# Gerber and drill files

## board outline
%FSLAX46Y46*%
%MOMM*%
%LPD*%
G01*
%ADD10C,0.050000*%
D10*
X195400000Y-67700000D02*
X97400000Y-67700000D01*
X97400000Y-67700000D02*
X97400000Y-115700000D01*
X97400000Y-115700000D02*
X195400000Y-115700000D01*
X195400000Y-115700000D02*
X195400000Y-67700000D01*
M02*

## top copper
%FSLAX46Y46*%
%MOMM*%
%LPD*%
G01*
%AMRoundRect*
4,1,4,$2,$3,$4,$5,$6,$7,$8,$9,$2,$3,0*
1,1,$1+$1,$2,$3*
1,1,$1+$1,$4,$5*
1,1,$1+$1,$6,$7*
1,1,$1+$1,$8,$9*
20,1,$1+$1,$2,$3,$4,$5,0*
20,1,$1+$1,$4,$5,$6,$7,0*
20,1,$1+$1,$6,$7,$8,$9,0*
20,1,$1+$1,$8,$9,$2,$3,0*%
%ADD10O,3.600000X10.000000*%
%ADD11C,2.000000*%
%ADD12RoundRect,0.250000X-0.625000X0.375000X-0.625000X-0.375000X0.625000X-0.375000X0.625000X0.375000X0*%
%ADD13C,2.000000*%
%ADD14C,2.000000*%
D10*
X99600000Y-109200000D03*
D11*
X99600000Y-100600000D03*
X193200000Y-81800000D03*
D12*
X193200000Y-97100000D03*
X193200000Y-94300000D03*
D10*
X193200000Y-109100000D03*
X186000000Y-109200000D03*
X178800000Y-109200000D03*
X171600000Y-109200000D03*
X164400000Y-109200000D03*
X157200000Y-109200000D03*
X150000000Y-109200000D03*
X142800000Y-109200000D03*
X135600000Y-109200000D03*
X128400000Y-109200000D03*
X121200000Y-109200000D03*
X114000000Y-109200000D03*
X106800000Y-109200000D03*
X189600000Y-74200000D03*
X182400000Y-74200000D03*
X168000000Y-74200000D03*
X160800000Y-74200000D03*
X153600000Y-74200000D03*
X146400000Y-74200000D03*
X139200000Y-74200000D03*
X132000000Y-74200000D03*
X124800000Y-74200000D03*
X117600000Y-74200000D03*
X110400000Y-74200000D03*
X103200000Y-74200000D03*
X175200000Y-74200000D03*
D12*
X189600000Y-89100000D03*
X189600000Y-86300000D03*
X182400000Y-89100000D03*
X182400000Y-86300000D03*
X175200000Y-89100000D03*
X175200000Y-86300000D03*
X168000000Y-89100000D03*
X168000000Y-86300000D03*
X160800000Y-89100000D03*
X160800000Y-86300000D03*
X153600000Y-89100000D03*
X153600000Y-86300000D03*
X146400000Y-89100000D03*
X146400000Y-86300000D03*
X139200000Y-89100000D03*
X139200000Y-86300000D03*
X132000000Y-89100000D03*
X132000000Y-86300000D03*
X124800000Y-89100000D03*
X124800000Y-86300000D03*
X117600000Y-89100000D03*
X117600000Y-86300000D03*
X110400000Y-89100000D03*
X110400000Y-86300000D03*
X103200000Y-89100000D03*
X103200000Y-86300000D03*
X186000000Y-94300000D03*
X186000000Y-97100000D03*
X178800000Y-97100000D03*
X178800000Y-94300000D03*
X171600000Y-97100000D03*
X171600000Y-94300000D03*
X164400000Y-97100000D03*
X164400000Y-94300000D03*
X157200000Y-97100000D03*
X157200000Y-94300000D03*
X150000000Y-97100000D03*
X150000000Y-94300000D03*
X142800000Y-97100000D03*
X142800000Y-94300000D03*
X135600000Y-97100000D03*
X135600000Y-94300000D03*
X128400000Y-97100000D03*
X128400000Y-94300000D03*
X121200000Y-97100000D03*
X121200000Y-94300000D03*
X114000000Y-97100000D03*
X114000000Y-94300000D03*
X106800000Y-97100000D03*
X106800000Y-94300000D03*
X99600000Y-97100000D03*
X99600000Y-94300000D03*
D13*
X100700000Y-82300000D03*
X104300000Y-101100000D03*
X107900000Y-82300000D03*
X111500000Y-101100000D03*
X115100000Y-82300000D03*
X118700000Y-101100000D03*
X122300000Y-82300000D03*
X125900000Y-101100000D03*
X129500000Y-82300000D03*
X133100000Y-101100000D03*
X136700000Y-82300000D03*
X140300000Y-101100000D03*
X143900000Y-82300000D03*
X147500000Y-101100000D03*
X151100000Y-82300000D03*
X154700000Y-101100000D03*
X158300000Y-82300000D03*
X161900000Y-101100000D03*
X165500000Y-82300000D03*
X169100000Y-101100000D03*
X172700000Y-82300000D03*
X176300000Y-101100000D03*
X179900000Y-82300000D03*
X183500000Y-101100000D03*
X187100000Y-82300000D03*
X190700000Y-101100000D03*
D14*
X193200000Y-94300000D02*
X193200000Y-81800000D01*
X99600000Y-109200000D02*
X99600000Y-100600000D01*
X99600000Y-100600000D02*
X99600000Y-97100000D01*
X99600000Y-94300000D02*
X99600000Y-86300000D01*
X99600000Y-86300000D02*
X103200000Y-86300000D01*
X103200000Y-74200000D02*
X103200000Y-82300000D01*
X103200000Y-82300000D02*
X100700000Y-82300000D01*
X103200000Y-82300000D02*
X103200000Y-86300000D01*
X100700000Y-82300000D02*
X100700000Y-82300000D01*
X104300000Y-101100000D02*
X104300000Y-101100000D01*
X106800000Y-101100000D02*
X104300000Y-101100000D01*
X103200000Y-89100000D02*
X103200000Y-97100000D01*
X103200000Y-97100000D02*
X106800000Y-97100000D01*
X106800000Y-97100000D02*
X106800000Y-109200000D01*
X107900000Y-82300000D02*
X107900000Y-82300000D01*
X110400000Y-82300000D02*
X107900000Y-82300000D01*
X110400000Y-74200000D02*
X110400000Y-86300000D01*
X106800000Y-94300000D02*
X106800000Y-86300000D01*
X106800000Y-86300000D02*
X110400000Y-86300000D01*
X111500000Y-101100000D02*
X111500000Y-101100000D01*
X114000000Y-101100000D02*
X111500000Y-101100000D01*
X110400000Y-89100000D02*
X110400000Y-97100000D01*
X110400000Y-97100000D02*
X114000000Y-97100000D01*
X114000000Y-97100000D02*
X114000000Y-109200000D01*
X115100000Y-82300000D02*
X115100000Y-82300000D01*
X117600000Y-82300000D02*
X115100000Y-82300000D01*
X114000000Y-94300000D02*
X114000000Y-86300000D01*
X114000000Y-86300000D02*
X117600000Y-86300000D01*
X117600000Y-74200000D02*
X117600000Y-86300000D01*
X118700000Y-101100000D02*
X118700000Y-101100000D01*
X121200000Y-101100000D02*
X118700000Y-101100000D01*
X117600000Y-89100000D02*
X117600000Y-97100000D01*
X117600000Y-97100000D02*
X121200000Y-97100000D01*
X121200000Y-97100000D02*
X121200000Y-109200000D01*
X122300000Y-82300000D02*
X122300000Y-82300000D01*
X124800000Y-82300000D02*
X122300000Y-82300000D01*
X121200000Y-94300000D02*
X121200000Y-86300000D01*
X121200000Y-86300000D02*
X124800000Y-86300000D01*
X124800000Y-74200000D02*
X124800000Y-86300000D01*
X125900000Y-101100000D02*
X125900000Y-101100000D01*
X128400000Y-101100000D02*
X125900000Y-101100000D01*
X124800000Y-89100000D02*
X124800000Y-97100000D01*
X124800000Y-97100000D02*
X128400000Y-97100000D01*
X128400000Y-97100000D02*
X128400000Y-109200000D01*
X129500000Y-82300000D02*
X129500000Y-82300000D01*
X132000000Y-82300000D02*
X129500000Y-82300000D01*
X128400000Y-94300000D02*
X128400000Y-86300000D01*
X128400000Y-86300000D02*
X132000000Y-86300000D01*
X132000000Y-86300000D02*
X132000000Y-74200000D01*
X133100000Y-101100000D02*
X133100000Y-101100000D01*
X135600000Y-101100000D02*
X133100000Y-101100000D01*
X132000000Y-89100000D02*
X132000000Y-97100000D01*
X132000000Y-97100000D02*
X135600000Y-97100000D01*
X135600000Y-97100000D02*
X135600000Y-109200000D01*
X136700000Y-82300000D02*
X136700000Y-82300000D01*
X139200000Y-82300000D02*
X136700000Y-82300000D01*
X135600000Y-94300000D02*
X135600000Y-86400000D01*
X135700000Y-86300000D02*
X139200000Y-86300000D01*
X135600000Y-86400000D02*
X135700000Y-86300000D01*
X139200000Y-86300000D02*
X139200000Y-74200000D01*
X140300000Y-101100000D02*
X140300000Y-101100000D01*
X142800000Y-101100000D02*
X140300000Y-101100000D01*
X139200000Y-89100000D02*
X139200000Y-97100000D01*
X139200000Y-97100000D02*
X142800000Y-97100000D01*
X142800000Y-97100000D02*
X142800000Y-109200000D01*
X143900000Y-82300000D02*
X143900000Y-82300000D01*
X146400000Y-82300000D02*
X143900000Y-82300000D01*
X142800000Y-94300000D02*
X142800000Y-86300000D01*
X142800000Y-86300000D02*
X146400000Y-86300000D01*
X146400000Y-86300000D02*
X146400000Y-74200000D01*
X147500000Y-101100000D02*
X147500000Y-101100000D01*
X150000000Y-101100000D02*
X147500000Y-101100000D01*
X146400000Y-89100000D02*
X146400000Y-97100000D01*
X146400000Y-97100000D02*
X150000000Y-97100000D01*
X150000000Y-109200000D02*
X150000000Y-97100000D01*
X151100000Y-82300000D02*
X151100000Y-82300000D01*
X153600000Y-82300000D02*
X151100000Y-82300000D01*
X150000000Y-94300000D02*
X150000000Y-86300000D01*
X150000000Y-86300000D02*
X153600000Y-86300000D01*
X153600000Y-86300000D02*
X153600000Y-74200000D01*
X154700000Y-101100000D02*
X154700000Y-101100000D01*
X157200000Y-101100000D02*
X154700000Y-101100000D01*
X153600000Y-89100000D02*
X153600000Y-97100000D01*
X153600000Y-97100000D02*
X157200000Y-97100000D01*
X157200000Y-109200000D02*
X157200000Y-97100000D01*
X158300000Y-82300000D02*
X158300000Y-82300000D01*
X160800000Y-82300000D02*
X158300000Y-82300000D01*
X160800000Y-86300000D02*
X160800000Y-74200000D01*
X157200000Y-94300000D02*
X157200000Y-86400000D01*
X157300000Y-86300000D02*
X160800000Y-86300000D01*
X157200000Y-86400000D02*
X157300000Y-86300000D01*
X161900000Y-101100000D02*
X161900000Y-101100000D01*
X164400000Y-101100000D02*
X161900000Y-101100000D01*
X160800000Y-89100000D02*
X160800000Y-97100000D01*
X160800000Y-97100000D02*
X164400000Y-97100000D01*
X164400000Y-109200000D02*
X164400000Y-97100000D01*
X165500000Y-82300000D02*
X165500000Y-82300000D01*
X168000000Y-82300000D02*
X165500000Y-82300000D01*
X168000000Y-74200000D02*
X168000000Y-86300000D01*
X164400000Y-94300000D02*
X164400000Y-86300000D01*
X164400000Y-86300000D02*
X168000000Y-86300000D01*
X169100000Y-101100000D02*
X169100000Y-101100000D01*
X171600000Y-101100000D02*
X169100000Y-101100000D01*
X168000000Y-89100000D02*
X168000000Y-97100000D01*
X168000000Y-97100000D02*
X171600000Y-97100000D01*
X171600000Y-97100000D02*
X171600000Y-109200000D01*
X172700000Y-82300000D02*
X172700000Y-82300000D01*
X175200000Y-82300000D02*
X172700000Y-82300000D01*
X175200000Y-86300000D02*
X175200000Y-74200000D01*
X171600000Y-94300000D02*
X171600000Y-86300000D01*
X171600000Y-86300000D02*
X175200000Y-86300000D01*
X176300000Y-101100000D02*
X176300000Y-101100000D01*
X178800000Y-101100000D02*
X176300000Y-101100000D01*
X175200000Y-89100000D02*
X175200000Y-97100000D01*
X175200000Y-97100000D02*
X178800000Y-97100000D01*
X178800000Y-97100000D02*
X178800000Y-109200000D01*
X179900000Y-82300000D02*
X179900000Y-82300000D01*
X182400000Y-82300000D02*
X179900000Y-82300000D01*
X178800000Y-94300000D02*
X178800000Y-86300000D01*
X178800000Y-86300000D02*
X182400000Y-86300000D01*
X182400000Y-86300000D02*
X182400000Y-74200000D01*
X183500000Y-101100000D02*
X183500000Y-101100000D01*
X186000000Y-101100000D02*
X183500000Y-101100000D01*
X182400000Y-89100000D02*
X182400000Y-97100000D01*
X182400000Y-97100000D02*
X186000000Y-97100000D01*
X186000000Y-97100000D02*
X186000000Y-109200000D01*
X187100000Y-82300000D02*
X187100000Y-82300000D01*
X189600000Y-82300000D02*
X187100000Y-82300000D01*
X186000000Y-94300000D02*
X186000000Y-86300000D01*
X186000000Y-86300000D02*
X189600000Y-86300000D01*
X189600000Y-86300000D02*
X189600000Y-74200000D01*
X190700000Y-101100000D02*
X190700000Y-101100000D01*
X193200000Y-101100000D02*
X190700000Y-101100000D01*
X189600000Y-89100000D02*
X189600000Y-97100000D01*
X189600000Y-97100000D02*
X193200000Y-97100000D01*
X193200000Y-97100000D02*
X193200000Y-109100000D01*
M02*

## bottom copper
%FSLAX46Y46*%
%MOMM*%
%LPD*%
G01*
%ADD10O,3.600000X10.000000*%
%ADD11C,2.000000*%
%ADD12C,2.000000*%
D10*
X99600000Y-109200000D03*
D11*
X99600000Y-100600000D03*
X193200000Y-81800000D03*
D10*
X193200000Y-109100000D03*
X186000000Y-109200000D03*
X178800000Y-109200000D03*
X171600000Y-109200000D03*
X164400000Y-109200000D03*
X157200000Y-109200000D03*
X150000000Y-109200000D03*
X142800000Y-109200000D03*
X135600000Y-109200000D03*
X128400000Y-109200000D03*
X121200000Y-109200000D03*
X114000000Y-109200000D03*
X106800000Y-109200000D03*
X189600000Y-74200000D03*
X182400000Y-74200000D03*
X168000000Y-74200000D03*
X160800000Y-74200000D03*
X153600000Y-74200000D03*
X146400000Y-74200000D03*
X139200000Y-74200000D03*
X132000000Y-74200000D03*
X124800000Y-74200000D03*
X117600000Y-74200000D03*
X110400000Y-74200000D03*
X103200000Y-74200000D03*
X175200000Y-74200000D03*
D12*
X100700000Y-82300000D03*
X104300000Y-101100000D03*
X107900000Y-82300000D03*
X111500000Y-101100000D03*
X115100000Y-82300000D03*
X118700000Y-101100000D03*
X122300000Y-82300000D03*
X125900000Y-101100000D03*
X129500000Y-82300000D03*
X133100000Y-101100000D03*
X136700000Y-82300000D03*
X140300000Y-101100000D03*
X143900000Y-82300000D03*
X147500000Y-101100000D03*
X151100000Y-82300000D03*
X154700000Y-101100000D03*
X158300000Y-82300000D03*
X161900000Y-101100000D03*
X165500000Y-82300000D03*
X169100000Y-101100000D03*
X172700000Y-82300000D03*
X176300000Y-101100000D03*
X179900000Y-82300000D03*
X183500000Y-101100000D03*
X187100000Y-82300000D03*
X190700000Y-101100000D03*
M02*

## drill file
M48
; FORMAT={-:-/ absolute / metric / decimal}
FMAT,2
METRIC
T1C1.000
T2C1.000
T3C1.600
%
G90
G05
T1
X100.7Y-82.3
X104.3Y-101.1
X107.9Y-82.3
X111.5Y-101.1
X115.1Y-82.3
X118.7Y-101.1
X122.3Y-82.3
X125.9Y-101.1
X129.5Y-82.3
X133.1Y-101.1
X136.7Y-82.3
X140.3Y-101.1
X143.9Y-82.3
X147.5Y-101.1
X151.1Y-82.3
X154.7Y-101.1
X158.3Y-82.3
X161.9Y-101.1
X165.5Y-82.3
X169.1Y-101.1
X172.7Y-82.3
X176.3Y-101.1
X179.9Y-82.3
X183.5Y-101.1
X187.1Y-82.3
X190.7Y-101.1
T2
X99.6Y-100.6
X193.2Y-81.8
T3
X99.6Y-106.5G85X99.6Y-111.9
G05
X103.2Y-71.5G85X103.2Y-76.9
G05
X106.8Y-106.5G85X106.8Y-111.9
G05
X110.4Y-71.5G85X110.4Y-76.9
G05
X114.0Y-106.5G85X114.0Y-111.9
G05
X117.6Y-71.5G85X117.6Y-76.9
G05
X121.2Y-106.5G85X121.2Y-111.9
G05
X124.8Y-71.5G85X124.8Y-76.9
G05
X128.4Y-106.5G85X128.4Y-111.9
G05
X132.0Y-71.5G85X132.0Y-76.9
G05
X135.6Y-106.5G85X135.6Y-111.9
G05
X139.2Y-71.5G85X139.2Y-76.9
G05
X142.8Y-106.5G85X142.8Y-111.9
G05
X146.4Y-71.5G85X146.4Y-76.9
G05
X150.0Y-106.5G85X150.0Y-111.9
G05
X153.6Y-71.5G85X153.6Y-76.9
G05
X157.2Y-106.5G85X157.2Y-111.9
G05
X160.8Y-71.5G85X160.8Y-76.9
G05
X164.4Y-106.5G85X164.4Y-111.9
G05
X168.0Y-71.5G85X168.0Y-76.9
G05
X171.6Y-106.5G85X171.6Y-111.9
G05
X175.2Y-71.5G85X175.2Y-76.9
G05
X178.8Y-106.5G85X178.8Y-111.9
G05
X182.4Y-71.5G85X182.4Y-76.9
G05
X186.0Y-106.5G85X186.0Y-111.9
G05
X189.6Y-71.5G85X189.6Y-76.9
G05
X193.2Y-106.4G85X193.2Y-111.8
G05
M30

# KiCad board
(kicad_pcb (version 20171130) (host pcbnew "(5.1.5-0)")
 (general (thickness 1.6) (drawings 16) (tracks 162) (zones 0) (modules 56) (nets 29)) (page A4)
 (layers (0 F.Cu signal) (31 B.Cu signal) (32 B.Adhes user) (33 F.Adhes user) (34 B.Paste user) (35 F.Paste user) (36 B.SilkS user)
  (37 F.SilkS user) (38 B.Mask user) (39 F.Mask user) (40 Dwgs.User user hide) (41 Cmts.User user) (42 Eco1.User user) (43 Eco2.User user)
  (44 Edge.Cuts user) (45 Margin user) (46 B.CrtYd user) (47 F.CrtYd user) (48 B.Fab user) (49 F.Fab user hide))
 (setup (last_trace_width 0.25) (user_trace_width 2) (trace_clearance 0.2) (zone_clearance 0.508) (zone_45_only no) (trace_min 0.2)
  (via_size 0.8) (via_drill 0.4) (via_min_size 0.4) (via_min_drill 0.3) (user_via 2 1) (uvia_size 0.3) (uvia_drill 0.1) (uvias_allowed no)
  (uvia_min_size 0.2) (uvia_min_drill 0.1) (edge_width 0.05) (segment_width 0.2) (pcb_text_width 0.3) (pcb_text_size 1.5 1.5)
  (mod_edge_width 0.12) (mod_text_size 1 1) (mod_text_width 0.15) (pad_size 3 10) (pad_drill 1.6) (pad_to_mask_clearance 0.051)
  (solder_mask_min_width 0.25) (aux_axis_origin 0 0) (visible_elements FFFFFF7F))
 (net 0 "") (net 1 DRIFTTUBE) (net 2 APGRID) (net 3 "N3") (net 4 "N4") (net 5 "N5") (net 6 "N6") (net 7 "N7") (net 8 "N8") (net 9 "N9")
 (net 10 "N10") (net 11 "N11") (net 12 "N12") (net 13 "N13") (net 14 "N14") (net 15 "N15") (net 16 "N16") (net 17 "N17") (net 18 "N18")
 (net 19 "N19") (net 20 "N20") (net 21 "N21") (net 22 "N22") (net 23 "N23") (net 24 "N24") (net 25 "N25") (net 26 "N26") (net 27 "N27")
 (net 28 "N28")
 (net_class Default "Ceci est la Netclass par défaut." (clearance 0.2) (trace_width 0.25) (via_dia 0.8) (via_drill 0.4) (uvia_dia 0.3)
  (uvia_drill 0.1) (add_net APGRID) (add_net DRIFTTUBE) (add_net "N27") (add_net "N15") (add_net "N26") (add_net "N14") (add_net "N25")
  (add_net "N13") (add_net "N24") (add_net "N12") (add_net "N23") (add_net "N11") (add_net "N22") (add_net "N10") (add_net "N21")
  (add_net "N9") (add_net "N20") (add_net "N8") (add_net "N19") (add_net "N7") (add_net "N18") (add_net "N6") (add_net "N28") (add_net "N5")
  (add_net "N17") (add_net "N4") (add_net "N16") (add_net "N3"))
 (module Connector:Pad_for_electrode (layer F.Cu) (at 99.6 109.3)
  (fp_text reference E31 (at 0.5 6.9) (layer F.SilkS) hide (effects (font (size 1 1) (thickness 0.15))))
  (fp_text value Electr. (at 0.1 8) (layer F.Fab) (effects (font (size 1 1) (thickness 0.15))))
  (pad 1 thru_hole oval (at 0 -0.1) (size 3.6 10) (drill oval 1.6 7) (layers *.Cu *.Mask) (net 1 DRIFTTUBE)))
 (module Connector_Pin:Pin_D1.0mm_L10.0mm (layer F.Cu) (at 99.6 100.6)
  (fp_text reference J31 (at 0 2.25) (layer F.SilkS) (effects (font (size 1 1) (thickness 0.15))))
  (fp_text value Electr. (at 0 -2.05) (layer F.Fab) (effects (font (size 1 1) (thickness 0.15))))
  (pad 1 thru_hole circle (at 0 0) (size 2 2) (drill 1) (layers *.Cu *.Mask) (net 1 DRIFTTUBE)))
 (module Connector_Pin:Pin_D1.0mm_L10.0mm (layer F.Cu) (at 193.2 81.8)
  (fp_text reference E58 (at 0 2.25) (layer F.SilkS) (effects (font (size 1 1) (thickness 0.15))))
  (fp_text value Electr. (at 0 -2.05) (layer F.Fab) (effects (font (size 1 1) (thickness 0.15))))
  (pad 1 thru_hole circle (at 0 0) (size 2 2) (drill 1) (layers *.Cu *.Mask) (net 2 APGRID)))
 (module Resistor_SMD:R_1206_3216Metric (layer F.Cu) (at 193.2 95.7 270)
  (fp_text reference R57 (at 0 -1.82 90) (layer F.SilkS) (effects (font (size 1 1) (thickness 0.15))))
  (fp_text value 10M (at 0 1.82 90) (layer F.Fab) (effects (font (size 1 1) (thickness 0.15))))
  (pad 2 smd roundrect (at 1.4 0 270) (size 1.25 1.75) (layers F.Cu F.Paste F.Mask) (roundrect_rratio 0.2) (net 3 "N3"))
  (pad 1 smd roundrect (at -1.4 0 270) (size 1.25 1.75) (layers F.Cu F.Paste F.Mask) (roundrect_rratio 0.2) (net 2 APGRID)))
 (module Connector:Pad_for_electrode (layer F.Cu) (at 193.2 109.2)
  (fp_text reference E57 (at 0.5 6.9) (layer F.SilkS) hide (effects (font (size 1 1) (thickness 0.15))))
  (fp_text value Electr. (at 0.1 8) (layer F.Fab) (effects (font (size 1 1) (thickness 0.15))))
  (pad 1 thru_hole oval (at 0 -0.1) (size 3.6 10) (drill oval 1.6 7) (layers *.Cu *.Mask) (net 3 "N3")))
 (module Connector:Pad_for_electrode (layer F.Cu) (at 186 109.3)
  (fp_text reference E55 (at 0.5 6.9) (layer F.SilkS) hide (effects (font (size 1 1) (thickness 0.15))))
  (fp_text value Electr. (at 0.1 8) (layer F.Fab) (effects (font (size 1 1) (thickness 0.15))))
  (pad 1 thru_hole oval (at 0 -0.1) (size 3.6 10) (drill oval 1.6 7) (layers *.Cu *.Mask) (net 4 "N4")))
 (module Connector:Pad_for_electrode (layer F.Cu) (at 178.8 109.3)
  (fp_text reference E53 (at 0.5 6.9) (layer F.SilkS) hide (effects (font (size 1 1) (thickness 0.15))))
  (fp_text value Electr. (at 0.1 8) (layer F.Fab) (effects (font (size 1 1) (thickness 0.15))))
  (pad 1 thru_hole oval (at 0 -0.1) (size 3.6 10) (drill oval 1.6 7) (layers *.Cu *.Mask) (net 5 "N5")))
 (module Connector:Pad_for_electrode (layer F.Cu) (at 171.6 109.3)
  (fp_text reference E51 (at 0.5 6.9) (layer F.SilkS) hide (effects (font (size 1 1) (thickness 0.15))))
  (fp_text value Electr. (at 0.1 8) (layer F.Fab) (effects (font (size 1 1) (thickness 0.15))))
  (pad 1 thru_hole oval (at 0 -0.1) (size 3.6 10) (drill oval 1.6 7) (layers *.Cu *.Mask) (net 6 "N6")))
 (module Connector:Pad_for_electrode (layer F.Cu) (at 164.4 109.3)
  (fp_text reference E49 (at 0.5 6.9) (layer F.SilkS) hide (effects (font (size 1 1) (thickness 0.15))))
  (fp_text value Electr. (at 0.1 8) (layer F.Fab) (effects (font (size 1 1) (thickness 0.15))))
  (pad 1 thru_hole oval (at 0 -0.1) (size 3.6 10) (drill oval 1.6 7) (layers *.Cu *.Mask) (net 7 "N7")))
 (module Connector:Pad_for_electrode (layer F.Cu) (at 157.2 109.3)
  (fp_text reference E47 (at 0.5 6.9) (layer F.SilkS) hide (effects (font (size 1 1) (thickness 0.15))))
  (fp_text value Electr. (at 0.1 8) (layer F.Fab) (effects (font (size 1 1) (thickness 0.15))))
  (pad 1 thru_hole oval (at 0 -0.1) (size 3.6 10) (drill oval 1.6 7) (layers *.Cu *.Mask) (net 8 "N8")))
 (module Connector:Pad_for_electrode (layer F.Cu) (at 150 109.3)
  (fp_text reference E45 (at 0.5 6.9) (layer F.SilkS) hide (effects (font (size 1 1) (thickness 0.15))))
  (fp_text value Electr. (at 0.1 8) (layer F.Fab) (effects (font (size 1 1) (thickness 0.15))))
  (pad 1 thru_hole oval (at 0 -0.1) (size 3.6 10) (drill oval 1.6 7) (layers *.Cu *.Mask) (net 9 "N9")))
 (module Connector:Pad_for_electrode (layer F.Cu) (at 142.8 109.3)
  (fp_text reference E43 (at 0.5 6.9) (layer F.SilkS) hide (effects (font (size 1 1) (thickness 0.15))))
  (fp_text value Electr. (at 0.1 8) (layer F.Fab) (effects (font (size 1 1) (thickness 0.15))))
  (pad 1 thru_hole oval (at 0 -0.1) (size 3.6 10) (drill oval 1.6 7) (layers *.Cu *.Mask) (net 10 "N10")))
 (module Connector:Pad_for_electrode (layer F.Cu) (at 135.6 109.3)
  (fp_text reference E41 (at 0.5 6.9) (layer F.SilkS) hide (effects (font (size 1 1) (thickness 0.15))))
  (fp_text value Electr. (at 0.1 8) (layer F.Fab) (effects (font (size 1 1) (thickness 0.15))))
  (pad 1 thru_hole oval (at 0 -0.1) (size 3.6 10) (drill oval 1.6 7) (layers *.Cu *.Mask) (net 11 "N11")))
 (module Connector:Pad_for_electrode (layer F.Cu) (at 128.4 109.3)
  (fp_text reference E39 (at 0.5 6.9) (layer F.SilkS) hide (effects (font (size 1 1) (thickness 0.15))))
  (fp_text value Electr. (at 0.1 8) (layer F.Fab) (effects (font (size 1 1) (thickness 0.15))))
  (pad 1 thru_hole oval (at 0 -0.1) (size 3.6 10) (drill oval 1.6 7) (layers *.Cu *.Mask) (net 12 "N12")))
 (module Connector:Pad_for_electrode (layer F.Cu) (at 121.2 109.3)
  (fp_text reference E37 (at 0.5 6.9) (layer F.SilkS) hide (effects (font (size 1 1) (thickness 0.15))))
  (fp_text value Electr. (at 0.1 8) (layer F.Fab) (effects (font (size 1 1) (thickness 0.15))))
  (pad 1 thru_hole oval (at 0 -0.1) (size 3.6 10) (drill oval 1.6 7) (layers *.Cu *.Mask) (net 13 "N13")))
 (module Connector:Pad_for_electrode (layer F.Cu) (at 114 109.3)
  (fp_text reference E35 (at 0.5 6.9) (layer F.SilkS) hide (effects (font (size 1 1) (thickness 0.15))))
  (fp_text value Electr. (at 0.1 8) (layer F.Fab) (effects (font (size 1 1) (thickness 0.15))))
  (pad 1 thru_hole oval (at 0 -0.1) (size 3.6 10) (drill oval 1.6 7) (layers *.Cu *.Mask) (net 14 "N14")))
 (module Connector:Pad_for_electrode (layer F.Cu) (at 106.8 109.3)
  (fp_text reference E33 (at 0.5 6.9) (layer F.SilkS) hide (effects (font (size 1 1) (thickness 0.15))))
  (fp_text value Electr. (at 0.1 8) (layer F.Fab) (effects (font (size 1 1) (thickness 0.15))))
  (pad 1 thru_hole oval (at 0 -0.1) (size 3.6 10) (drill oval 1.6 7) (layers *.Cu *.Mask) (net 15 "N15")))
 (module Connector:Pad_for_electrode (layer F.Cu) (at 189.6 74.3)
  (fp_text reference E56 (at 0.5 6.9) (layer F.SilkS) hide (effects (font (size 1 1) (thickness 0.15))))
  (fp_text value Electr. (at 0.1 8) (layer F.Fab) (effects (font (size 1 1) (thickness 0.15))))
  (pad 1 thru_hole oval (at 0 -0.1) (size 3.6 10) (drill oval 1.6 7) (layers *.Cu *.Mask) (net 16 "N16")))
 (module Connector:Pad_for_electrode (layer F.Cu) (at 182.4 74.3)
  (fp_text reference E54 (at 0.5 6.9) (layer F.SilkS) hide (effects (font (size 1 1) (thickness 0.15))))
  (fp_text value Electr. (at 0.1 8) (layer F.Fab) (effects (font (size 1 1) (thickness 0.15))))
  (pad 1 thru_hole oval (at 0 -0.1) (size 3.6 10) (drill oval 1.6 7) (layers *.Cu *.Mask) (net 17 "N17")))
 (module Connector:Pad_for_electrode (layer F.Cu) (at 168 74.3)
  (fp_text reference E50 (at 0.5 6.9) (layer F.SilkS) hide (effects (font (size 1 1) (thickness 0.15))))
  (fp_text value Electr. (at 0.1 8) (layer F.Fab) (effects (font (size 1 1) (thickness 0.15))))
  (pad 1 thru_hole oval (at 0 -0.1) (size 3.6 10) (drill oval 1.6 7) (layers *.Cu *.Mask) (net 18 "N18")))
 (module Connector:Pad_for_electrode (layer F.Cu) (at 160.8 74.3)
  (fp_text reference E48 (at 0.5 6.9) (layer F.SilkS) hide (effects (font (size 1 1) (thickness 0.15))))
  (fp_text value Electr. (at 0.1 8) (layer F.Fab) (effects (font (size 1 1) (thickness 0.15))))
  (pad 1 thru_hole oval (at 0 -0.1) (size 3.6 10) (drill oval 1.6 7) (layers *.Cu *.Mask) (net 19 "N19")))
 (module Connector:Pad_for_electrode (layer F.Cu) (at 153.6 74.3)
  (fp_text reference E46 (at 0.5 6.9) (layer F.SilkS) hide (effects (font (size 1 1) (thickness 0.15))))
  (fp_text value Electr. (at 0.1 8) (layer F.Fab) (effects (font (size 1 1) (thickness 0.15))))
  (pad 1 thru_hole oval (at 0 -0.1) (size 3.6 10) (drill oval 1.6 7) (layers *.Cu *.Mask) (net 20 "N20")))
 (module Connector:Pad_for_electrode (layer F.Cu) (at 146.4 74.3)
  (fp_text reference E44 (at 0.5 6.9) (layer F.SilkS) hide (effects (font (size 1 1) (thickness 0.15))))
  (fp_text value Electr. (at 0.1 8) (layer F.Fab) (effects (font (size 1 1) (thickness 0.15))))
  (pad 1 thru_hole oval (at 0 -0.1) (size 3.6 10) (drill oval 1.6 7) (layers *.Cu *.Mask) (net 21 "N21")))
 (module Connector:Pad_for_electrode (layer F.Cu) (at 139.2 74.3)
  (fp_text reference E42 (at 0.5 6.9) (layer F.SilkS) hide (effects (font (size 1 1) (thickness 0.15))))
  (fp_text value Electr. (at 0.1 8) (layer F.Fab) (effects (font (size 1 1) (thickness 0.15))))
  (pad 1 thru_hole oval (at 0 -0.1) (size 3.6 10) (drill oval 1.6 7) (layers *.Cu *.Mask) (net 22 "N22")))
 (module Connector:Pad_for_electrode (layer F.Cu) (at 132 74.3)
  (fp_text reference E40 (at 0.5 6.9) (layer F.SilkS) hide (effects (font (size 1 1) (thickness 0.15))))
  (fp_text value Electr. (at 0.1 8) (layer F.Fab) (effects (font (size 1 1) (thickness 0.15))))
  (pad 1 thru_hole oval (at 0 -0.1) (size 3.6 10) (drill oval 1.6 7) (layers *.Cu *.Mask) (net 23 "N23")))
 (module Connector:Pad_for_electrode (layer F.Cu) (at 124.8 74.3)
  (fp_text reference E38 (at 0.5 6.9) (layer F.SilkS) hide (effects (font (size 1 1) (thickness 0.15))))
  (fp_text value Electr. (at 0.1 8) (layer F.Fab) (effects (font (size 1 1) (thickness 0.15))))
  (pad 1 thru_hole oval (at 0 -0.1) (size 3.6 10) (drill oval 1.6 7) (layers *.Cu *.Mask) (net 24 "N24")))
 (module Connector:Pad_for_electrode (layer F.Cu) (at 117.6 74.3)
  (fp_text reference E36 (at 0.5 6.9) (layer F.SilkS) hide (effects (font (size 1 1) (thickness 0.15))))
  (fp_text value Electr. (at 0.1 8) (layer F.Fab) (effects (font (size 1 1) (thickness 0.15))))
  (pad 1 thru_hole oval (at 0 -0.1) (size 3.6 10) (drill oval 1.6 7) (layers *.Cu *.Mask) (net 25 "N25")))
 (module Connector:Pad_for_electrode (layer F.Cu) (at 110.4 74.3)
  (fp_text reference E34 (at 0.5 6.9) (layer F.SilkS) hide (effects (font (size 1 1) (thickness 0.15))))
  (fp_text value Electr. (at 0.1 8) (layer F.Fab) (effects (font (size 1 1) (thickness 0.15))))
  (pad 1 thru_hole oval (at 0 -0.1) (size 3.6 10) (drill oval 1.6 7) (layers *.Cu *.Mask) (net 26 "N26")))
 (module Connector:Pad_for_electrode (layer F.Cu) (at 103.2 74.3)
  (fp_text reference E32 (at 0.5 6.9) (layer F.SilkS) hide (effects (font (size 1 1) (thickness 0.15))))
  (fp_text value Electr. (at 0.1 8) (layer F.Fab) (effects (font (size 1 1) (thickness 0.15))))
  (pad 1 thru_hole oval (at 0 -0.1) (size 3.6 10) (drill oval 1.6 7) (layers *.Cu *.Mask) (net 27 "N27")))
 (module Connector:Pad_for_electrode (layer F.Cu) (at 175.2 74.3)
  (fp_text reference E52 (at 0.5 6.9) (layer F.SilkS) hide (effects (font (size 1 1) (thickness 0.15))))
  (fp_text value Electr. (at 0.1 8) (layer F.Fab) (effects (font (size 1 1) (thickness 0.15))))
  (pad 1 thru_hole oval (at 0 -0.1) (size 3.6 10) (drill oval 1.6 7) (layers *.Cu *.Mask) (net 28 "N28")))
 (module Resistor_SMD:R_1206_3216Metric (layer F.Cu) (at 189.6 87.7 270)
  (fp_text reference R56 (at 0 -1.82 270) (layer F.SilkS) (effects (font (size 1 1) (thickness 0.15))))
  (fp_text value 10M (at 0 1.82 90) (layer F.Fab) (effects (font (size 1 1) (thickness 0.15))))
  (pad 2 smd roundrect (at 1.4 0 270) (size 1.25 1.75) (layers F.Cu F.Paste F.Mask) (roundrect_rratio 0.2) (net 3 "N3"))
  (pad 1 smd roundrect (at -1.4 0 270) (size 1.25 1.75) (layers F.Cu F.Paste F.Mask) (roundrect_rratio 0.2) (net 16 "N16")))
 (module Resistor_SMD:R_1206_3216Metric (layer F.Cu) (at 182.4 87.7 270)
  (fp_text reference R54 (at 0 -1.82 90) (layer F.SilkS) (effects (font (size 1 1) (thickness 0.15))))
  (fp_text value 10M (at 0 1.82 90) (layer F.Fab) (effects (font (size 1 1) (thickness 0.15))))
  (pad 2 smd roundrect (at 1.4 0 270) (size 1.25 1.75) (layers F.Cu F.Paste F.Mask) (roundrect_rratio 0.2) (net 4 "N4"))
  (pad 1 smd roundrect (at -1.4 0 270) (size 1.25 1.75) (layers F.Cu F.Paste F.Mask) (roundrect_rratio 0.2) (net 17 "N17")))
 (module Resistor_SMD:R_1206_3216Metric (layer F.Cu) (at 175.2 87.7 270)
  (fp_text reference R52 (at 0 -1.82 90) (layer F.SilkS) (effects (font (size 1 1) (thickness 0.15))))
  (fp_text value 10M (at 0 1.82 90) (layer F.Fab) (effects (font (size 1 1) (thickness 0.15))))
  (pad 2 smd roundrect (at 1.4 0 270) (size 1.25 1.75) (layers F.Cu F.Paste F.Mask) (roundrect_rratio 0.2) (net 5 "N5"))
  (pad 1 smd roundrect (at -1.4 0 270) (size 1.25 1.75) (layers F.Cu F.Paste F.Mask) (roundrect_rratio 0.2) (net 28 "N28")))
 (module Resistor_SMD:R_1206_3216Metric (layer F.Cu) (at 168 87.7 270)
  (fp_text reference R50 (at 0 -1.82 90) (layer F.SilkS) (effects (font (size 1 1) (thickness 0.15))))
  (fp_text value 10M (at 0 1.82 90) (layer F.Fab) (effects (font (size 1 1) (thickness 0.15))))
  (pad 2 smd roundrect (at 1.4 0 270) (size 1.25 1.75) (layers F.Cu F.Paste F.Mask) (roundrect_rratio 0.2) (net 6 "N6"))
  (pad 1 smd roundrect (at -1.4 0 270) (size 1.25 1.75) (layers F.Cu F.Paste F.Mask) (roundrect_rratio 0.2) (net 18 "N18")))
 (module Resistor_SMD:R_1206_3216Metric (layer F.Cu) (at 160.8 87.7 270)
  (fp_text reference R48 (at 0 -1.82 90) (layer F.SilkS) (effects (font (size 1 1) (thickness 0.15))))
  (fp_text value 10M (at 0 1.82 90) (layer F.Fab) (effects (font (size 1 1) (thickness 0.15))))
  (pad 2 smd roundrect (at 1.4 0 270) (size 1.25 1.75) (layers F.Cu F.Paste F.Mask) (roundrect_rratio 0.2) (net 7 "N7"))
  (pad 1 smd roundrect (at -1.4 0 270) (size 1.25 1.75) (layers F.Cu F.Paste F.Mask) (roundrect_rratio 0.2) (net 19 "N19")))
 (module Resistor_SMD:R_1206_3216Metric (layer F.Cu) (at 153.6 87.7 270)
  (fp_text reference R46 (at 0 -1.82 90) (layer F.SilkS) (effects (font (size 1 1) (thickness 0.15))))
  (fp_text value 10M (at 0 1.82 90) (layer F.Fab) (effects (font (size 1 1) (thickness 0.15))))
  (pad 2 smd roundrect (at 1.4 0 270) (size 1.25 1.75) (layers F.Cu F.Paste F.Mask) (roundrect_rratio 0.2) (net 8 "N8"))
  (pad 1 smd roundrect (at -1.4 0 270) (size 1.25 1.75) (layers F.Cu F.Paste F.Mask) (roundrect_rratio 0.2) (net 20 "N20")))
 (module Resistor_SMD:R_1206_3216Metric (layer F.Cu) (at 146.4 87.7 270)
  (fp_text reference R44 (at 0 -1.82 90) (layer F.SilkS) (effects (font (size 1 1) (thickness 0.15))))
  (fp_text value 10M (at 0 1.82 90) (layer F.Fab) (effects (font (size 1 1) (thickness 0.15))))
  (pad 2 smd roundrect (at 1.4 0 270) (size 1.25 1.75) (layers F.Cu F.Paste F.Mask) (roundrect_rratio 0.2) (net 9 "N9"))
  (pad 1 smd roundrect (at -1.4 0 270) (size 1.25 1.75) (layers F.Cu F.Paste F.Mask) (roundrect_rratio 0.2) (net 21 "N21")))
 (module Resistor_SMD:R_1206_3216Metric (layer F.Cu) (at 139.2 87.7 270)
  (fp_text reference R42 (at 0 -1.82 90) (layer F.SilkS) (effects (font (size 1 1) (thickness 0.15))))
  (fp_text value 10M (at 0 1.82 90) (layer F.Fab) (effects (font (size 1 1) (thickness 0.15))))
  (pad 2 smd roundrect (at 1.4 0 270) (size 1.25 1.75) (layers F.Cu F.Paste F.Mask) (roundrect_rratio 0.2) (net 10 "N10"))
  (pad 1 smd roundrect (at -1.4 0 270) (size 1.25 1.75) (layers F.Cu F.Paste F.Mask) (roundrect_rratio 0.2) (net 22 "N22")))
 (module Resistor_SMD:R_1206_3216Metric (layer F.Cu) (at 132 87.7 270)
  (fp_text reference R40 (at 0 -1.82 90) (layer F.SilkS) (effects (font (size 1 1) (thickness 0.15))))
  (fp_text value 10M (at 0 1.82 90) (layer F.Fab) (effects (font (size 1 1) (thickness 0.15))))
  (pad 2 smd roundrect (at 1.4 0 270) (size 1.25 1.75) (layers F.Cu F.Paste F.Mask) (roundrect_rratio 0.2) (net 11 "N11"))
  (pad 1 smd roundrect (at -1.4 0 270) (size 1.25 1.75) (layers F.Cu F.Paste F.Mask) (roundrect_rratio 0.2) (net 23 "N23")))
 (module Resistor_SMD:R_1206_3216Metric (layer F.Cu) (at 124.8 87.7 270)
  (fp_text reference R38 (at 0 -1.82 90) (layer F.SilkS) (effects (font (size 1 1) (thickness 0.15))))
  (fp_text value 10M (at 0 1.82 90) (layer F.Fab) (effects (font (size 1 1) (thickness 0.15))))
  (pad 2 smd roundrect (at 1.4 0 270) (size 1.25 1.75) (layers F.Cu F.Paste F.Mask) (roundrect_rratio 0.2) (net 12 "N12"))
  (pad 1 smd roundrect (at -1.4 0 270) (size 1.25 1.75) (layers F.Cu F.Paste F.Mask) (roundrect_rratio 0.2) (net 24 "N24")))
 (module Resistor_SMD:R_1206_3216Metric (layer F.Cu) (at 117.6 87.7 270)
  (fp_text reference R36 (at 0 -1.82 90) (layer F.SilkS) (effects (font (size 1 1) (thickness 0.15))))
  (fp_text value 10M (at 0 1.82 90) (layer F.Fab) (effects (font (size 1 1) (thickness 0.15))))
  (pad 2 smd roundrect (at 1.4 0 270) (size 1.25 1.75) (layers F.Cu F.Paste F.Mask) (roundrect_rratio 0.2) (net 13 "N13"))
  (pad 1 smd roundrect (at -1.4 0 270) (size 1.25 1.75) (layers F.Cu F.Paste F.Mask) (roundrect_rratio 0.2) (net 25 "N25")))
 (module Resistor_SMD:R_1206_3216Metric (layer F.Cu) (at 110.4 87.7 270)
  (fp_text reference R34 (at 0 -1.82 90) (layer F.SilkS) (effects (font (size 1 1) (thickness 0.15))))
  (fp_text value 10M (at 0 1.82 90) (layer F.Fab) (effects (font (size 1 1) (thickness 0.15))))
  (pad 2 smd roundrect (at 1.4 0 270) (size 1.25 1.75) (layers F.Cu F.Paste F.Mask) (roundrect_rratio 0.2) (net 14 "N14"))
  (pad 1 smd roundrect (at -1.4 0 270) (size 1.25 1.75) (layers F.Cu F.Paste F.Mask) (roundrect_rratio 0.2) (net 26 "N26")))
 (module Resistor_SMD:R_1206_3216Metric (layer F.Cu) (at 103.2 87.7 270)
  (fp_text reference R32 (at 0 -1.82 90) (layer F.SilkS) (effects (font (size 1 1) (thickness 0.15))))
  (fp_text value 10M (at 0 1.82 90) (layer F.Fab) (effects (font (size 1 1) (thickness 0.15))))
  (pad 2 smd roundrect (at 1.4 0 270) (size 1.25 1.75) (layers F.Cu F.Paste F.Mask) (roundrect_rratio 0.2) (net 15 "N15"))
  (pad 1 smd roundrect (at -1.4 0 270) (size 1.25 1.75) (layers F.Cu F.Paste F.Mask) (roundrect_rratio 0.2) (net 27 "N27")))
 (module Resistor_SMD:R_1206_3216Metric (layer F.Cu) (at 186 95.7 270)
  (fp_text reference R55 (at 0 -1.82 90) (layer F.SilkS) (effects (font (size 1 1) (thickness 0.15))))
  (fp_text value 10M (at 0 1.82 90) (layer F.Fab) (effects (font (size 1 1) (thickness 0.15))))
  (pad 1 smd roundrect (at -1.4 0 270) (size 1.25 1.75) (layers F.Cu F.Paste F.Mask) (roundrect_rratio 0.2) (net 16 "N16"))
  (pad 2 smd roundrect (at 1.4 0 270) (size 1.25 1.75) (layers F.Cu F.Paste F.Mask) (roundrect_rratio 0.2) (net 4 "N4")))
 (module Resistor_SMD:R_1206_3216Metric (layer F.Cu) (at 178.8 95.7 270)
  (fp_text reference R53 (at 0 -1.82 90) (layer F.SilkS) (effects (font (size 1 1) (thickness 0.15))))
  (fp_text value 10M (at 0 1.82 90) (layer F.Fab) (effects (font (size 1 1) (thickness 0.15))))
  (pad 2 smd roundrect (at 1.4 0 270) (size 1.25 1.75) (layers F.Cu F.Paste F.Mask) (roundrect_rratio 0.2) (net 5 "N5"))
  (pad 1 smd roundrect (at -1.4 0 270) (size 1.25 1.75) (layers F.Cu F.Paste F.Mask) (roundrect_rratio 0.2) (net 17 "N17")))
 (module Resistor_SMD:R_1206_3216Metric (layer F.Cu) (at 171.6 95.7 270)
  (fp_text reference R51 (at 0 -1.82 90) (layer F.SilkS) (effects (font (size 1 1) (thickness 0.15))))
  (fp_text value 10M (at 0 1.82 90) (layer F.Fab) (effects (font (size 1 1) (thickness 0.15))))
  (pad 2 smd roundrect (at 1.4 0 270) (size 1.25 1.75) (layers F.Cu F.Paste F.Mask) (roundrect_rratio 0.2) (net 6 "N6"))
  (pad 1 smd roundrect (at -1.4 0 270) (size 1.25 1.75) (layers F.Cu F.Paste F.Mask) (roundrect_rratio 0.2) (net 28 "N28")))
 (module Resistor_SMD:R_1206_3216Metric (layer F.Cu) (at 164.4 95.7 270)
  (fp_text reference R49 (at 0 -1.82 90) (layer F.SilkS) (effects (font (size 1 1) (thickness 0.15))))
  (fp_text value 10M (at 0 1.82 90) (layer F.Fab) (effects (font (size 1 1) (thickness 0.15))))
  (pad 2 smd roundrect (at 1.4 0 270) (size 1.25 1.75) (layers F.Cu F.Paste F.Mask) (roundrect_rratio 0.2) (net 7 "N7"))
  (pad 1 smd roundrect (at -1.4 0 270) (size 1.25 1.75) (layers F.Cu F.Paste F.Mask) (roundrect_rratio 0.2) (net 18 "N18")))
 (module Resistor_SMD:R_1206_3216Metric (layer F.Cu) (at 157.2 95.7 270)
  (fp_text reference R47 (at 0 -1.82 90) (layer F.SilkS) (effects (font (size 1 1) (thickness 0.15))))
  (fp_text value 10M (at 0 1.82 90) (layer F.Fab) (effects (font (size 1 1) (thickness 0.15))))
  (pad 2 smd roundrect (at 1.4 0 270) (size 1.25 1.75) (layers F.Cu F.Paste F.Mask) (roundrect_rratio 0.2) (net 8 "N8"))
  (pad 1 smd roundrect (at -1.4 0 270) (size 1.25 1.75) (layers F.Cu F.Paste F.Mask) (roundrect_rratio 0.2) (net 19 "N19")))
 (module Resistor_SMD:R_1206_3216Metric (layer F.Cu) (at 150 95.7 270)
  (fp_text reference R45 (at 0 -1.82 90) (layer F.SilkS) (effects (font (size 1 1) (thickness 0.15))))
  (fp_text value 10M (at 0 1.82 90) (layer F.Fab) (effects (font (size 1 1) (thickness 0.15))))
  (pad 2 smd roundrect (at 1.4 0 270) (size 1.25 1.75) (layers F.Cu F.Paste F.Mask) (roundrect_rratio 0.2) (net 9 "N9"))
  (pad 1 smd roundrect (at -1.4 0 270) (size 1.25 1.75) (layers F.Cu F.Paste F.Mask) (roundrect_rratio 0.2) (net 20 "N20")))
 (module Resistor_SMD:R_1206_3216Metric (layer F.Cu) (at 142.8 95.7 270)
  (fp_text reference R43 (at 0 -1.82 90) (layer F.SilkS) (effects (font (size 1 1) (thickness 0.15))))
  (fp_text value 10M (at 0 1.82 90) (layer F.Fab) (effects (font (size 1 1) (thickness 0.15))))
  (pad 2 smd roundrect (at 1.4 0 270) (size 1.25 1.75) (layers F.Cu F.Paste F.Mask) (roundrect_rratio 0.2) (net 10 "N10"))
  (pad 1 smd roundrect (at -1.4 0 270) (size 1.25 1.75) (layers F.Cu F.Paste F.Mask) (roundrect_rratio 0.2) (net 21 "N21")))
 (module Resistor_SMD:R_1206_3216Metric (layer F.Cu) (at 135.6 95.7 270)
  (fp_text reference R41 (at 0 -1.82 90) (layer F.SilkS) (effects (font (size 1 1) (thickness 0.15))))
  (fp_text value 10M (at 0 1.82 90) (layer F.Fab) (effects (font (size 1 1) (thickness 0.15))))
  (pad 2 smd roundrect (at 1.4 0 270) (size 1.25 1.75) (layers F.Cu F.Paste F.Mask) (roundrect_rratio 0.2) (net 11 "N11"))
  (pad 1 smd roundrect (at -1.4 0 270) (size 1.25 1.75) (layers F.Cu F.Paste F.Mask) (roundrect_rratio 0.2) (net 22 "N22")))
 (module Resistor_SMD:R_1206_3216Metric (layer F.Cu) (at 128.4 95.7 270)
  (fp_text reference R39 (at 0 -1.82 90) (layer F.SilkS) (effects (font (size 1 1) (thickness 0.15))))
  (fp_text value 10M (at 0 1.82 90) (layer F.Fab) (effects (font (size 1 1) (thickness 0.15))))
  (pad 2 smd roundrect (at 1.4 0 270) (size 1.25 1.75) (layers F.Cu F.Paste F.Mask) (roundrect_rratio 0.2) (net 12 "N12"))
  (pad 1 smd roundrect (at -1.4 0 270) (size 1.25 1.75) (layers F.Cu F.Paste F.Mask) (roundrect_rratio 0.2) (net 23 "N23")))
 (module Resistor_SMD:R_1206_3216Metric (layer F.Cu) (at 121.2 95.7 270)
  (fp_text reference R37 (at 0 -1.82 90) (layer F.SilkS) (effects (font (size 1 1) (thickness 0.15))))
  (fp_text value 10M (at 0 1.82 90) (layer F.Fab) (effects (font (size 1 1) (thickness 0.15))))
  (pad 2 smd roundrect (at 1.4 0 270) (size 1.25 1.75) (layers F.Cu F.Paste F.Mask) (roundrect_rratio 0.2) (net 13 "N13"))
  (pad 1 smd roundrect (at -1.4 0 270) (size 1.25 1.75) (layers F.Cu F.Paste F.Mask) (roundrect_rratio 0.2) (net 24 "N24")))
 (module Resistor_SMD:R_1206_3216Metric (layer F.Cu) (at 114 95.7 270)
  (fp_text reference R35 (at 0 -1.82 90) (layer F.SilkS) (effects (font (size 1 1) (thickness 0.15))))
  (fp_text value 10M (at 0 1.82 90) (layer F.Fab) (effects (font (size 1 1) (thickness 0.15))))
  (pad 2 smd roundrect (at 1.4 0 270) (size 1.25 1.75) (layers F.Cu F.Paste F.Mask) (roundrect_rratio 0.2) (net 14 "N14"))
  (pad 1 smd roundrect (at -1.4 0 270) (size 1.25 1.75) (layers F.Cu F.Paste F.Mask) (roundrect_rratio 0.2) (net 25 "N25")))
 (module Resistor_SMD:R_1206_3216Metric (layer F.Cu) (at 106.8 95.7 270)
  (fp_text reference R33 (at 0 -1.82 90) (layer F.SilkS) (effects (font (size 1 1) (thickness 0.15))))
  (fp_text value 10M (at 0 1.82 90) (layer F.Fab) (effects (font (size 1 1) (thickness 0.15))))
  (pad 2 smd roundrect (at 1.4 0 270) (size 1.25 1.75) (layers F.Cu F.Paste F.Mask) (roundrect_rratio 0.2) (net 15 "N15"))
  (pad 1 smd roundrect (at -1.4 0 270) (size 1.25 1.75) (layers F.Cu F.Paste F.Mask) (roundrect_rratio 0.2) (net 26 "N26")))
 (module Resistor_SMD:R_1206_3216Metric (layer F.Cu) (at 99.6 95.7 270)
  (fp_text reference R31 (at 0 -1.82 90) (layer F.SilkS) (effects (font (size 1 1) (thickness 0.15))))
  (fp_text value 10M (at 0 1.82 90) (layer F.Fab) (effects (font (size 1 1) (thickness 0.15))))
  (pad 2 smd roundrect (at 1.4 0 270) (size 1.25 1.75) (layers F.Cu F.Paste F.Mask) (roundrect_rratio 0.2) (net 1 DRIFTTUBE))
  (pad 1 smd roundrect (at -1.4 0 270) (size 1.25 1.75) (layers F.Cu F.Paste F.Mask) (roundrect_rratio 0.2) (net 27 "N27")))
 (gr_line (start 195.4 67.7) (end 97.4 67.7) (layer Edge.Cuts) (width 0.05))
 (gr_line (start 97.4 67.7) (end 97.4 115.7) (layer Edge.Cuts) (width 0.05))
 (gr_line (start 97.4 115.7) (end 195.4 115.7) (layer Edge.Cuts) (width 0.05))
 (gr_line (start 195.4 115.7) (end 195.4 67.7) (layer Edge.Cuts) (width 0.05))
 (segment (start 193.2 94.3) (end 193.2 81.8) (width 2) (layer F.Cu) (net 2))
 (segment (start 99.6 109.2) (end 99.6 100.6) (width 2) (layer F.Cu) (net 1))
 (segment (start 99.6 100.6) (end 99.6 97.1) (width 2) (layer F.Cu) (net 1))
 (segment (start 99.6 94.3) (end 99.6 86.3) (width 2) (layer F.Cu) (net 27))
 (segment (start 99.6 86.3) (end 103.2 86.3) (width 2) (layer F.Cu) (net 27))
 (segment (start 103.2 74.2) (end 103.2 82.3) (width 2) (layer F.Cu) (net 27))
 (segment (start 103.2 82.3) (end 100.7 82.3) (width 2) (layer F.Cu) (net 27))
 (segment (start 103.2 82.3) (end 103.2 86.3) (width 2) (layer F.Cu) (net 27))
 (segment (start 100.7 82.3) (end 100.7 82.3) (width 2) (layer F.Cu) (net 27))
 (via (at 100.7 82.3) (size 2) (drill 1) (layers F.Cu B.Cu) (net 27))
 (segment (start 104.3 101.1) (end 104.3 101.1) (width 2) (layer F.Cu) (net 15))
 (via (at 104.3 101.1) (size 2) (drill 1) (layers F.Cu B.Cu) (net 15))
 (segment (start 106.8 101.1) (end 104.3 101.1) (width 2) (layer F.Cu) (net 15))
 (segment (start 103.2 89.1) (end 103.2 97.1) (width 2) (layer F.Cu) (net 15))
 (segment (start 103.2 97.1) (end 106.8 97.1) (width 2) (layer F.Cu) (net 15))
 (segment (start 106.8 97.1) (end 106.8 109.2) (width 2) (layer F.Cu) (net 15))
 (segment (start 107.9 82.3) (end 107.9 82.3) (width 2) (layer F.Cu) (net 26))
 (via (at 107.9 82.3) (size 2) (drill 1) (layers F.Cu B.Cu) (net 26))
 (segment (start 110.4 82.3) (end 107.9 82.3) (width 2) (layer F.Cu) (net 26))
 (segment (start 110.4 74.2) (end 110.4 86.3) (width 2) (layer F.Cu) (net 26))
 (segment (start 106.8 94.3) (end 106.8 86.3) (width 2) (layer F.Cu) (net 26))
 (segment (start 106.8 86.3) (end 110.4 86.3) (width 2) (layer F.Cu) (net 26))
 (segment (start 111.5 101.1) (end 111.5 101.1) (width 2) (layer F.Cu) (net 14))
 (via (at 111.5 101.1) (size 2) (drill 1) (layers F.Cu B.Cu) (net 14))
 (segment (start 114 101.1) (end 111.5 101.1) (width 2) (layer F.Cu) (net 14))
 (segment (start 110.4 89.1) (end 110.4 97.1) (width 2) (layer F.Cu) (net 14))
 (segment (start 110.4 97.1) (end 114 97.1) (width 2) (layer F.Cu) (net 14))
 (segment (start 114 97.1) (end 114 109.2) (width 2) (layer F.Cu) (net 14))
 (segment (start 115.1 82.3) (end 115.1 82.3) (width 2) (layer F.Cu) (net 25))
 (via (at 115.1 82.3) (size 2) (drill 1) (layers F.Cu B.Cu) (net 25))
 (segment (start 117.6 82.3) (end 115.1 82.3) (width 2) (layer F.Cu) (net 25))
 (segment (start 114 94.3) (end 114 86.3) (width 2) (layer F.Cu) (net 25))
 (segment (start 114 86.3) (end 117.6 86.3) (width 2) (layer F.Cu) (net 25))
 (segment (start 117.6 74.2) (end 117.6 86.3) (width 2) (layer F.Cu) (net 25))
 (segment (start 118.7 101.1) (end 118.7 101.1) (width 2) (layer F.Cu) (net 13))
 (via (at 118.7 101.1) (size 2) (drill 1) (layers F.Cu B.Cu) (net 13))
 (segment (start 121.2 101.1) (end 118.7 101.1) (width 2) (layer F.Cu) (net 13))
 (segment (start 117.6 89.1) (end 117.6 97.1) (width 2) (layer F.Cu) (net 13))
 (segment (start 117.6 97.1) (end 121.2 97.1) (width 2) (layer F.Cu) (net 13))
 (segment (start 121.2 97.1) (end 121.2 109.2) (width 2) (layer F.Cu) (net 13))
 (segment (start 122.3 82.3) (end 122.3 82.3) (width 2) (layer F.Cu) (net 24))
 (via (at 122.3 82.3) (size 2) (drill 1) (layers F.Cu B.Cu) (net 24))
 (segment (start 124.8 82.3) (end 122.3 82.3) (width 2) (layer F.Cu) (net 24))
 (segment (start 121.2 94.3) (end 121.2 86.3) (width 2) (layer F.Cu) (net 24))
 (segment (start 121.2 86.3) (end 124.8 86.3) (width 2) (layer F.Cu) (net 24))
 (segment (start 124.8 74.2) (end 124.8 86.3) (width 2) (layer F.Cu) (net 24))
 (segment (start 125.9 101.1) (end 125.9 101.1) (width 2) (layer F.Cu) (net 12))
 (via (at 125.9 101.1) (size 2) (drill 1) (layers F.Cu B.Cu) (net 12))
 (segment (start 128.4 101.1) (end 125.9 101.1) (width 2) (layer F.Cu) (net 12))
 (segment (start 124.8 89.1) (end 124.8 97.1) (width 2) (layer F.Cu) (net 12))
 (segment (start 124.8 97.1) (end 128.4 97.1) (width 2) (layer F.Cu) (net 12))
 (segment (start 128.4 97.1) (end 128.4 109.2) (width 2) (layer F.Cu) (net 12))
 (segment (start 129.5 82.3) (end 129.5 82.3) (width 2) (layer F.Cu) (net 23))
 (via (at 129.5 82.3) (size 2) (drill 1) (layers F.Cu B.Cu) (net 23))
 (segment (start 132 82.3) (end 129.5 82.3) (width 2) (layer F.Cu) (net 23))
 (segment (start 128.4 94.3) (end 128.4 86.3) (width 2) (layer F.Cu) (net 23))
 (segment (start 128.4 86.3) (end 132 86.3) (width 2) (layer F.Cu) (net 23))
 (segment (start 132 86.3) (end 132 74.2) (width 2) (layer F.Cu) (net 23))
 (segment (start 133.1 101.1) (end 133.1 101.1) (width 2) (layer F.Cu) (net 11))
 (via (at 133.1 101.1) (size 2) (drill 1) (layers F.Cu B.Cu) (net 11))
 (segment (start 135.6 101.1) (end 133.1 101.1) (width 2) (layer F.Cu) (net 11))
 (segment (start 132 89.1) (end 132 97.1) (width 2) (layer F.Cu) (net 11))
 (segment (start 132 97.1) (end 135.6 97.1) (width 2) (layer F.Cu) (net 11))
 (segment (start 135.6 97.1) (end 135.6 109.2) (width 2) (layer F.Cu) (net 11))
 (segment (start 136.7 82.3) (end 136.7 82.3) (width 2) (layer F.Cu) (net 22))
 (via (at 136.7 82.3) (size 2) (drill 1) (layers F.Cu B.Cu) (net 22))
 (segment (start 139.2 82.3) (end 136.7 82.3) (width 2) (layer F.Cu) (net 22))
 (segment (start 135.6 94.3) (end 135.6 86.4) (width 2) (layer F.Cu) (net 22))
 (segment (start 135.7 86.3) (end 139.2 86.3) (width 2) (layer F.Cu) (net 22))
 (segment (start 135.6 86.4) (end 135.7 86.3) (width 2) (layer F.Cu) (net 22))
 (segment (start 139.2 86.3) (end 139.2 74.2) (width 2) (layer F.Cu) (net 22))
 (segment (start 140.3 101.1) (end 140.3 101.1) (width 2) (layer F.Cu) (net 10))
 (via (at 140.3 101.1) (size 2) (drill 1) (layers F.Cu B.Cu) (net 10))
 (segment (start 142.8 101.1) (end 140.3 101.1) (width 2) (layer F.Cu) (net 10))
 (segment (start 139.2 89.1) (end 139.2 97.1) (width 2) (layer F.Cu) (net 10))
 (segment (start 139.2 97.1) (end 142.8 97.1) (width 2) (layer F.Cu) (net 10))
 (segment (start 142.8 97.1) (end 142.8 109.2) (width 2) (layer F.Cu) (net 10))
 (segment (start 143.9 82.3) (end 143.9 82.3) (width 2) (layer F.Cu) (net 21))
 (via (at 143.9 82.3) (size 2) (drill 1) (layers F.Cu B.Cu) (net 21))
 (segment (start 146.4 82.3) (end 143.9 82.3) (width 2) (layer F.Cu) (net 21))
 (segment (start 142.8 94.3) (end 142.8 86.3) (width 2) (layer F.Cu) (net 21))
 (segment (start 142.8 86.3) (end 146.4 86.3) (width 2) (layer F.Cu) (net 21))
 (segment (start 146.4 86.3) (end 146.4 74.2) (width 2) (layer F.Cu) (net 21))
 (segment (start 147.5 101.1) (end 147.5 101.1) (width 2) (layer F.Cu) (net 9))
 (via (at 147.5 101.1) (size 2) (drill 1) (layers F.Cu B.Cu) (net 9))
 (segment (start 150 101.1) (end 147.5 101.1) (width 2) (layer F.Cu) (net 9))
 (segment (start 146.4 89.1) (end 146.4 97.1) (width 2) (layer F.Cu) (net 9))
 (segment (start 146.4 97.1) (end 150 97.1) (width 2) (layer F.Cu) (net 9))
 (segment (start 150 109.2) (end 150 97.1) (width 2) (layer F.Cu) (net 9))
 (segment (start 151.1 82.3) (end 151.1 82.3) (width 2) (layer F.Cu) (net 20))
 (via (at 151.1 82.3) (size 2) (drill 1) (layers F.Cu B.Cu) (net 20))
 (segment (start 153.6 82.3) (end 151.1 82.3) (width 2) (layer F.Cu) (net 20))
 (segment (start 150 94.3) (end 150 86.3) (width 2) (layer F.Cu) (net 20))
 (segment (start 150 86.3) (end 153.6 86.3) (width 2) (layer F.Cu) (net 20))
 (segment (start 153.6 86.3) (end 153.6 74.2) (width 2) (layer F.Cu) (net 20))
 (segment (start 154.7 101.1) (end 154.7 101.1) (width 2) (layer F.Cu) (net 8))
 (via (at 154.7 101.1) (size 2) (drill 1) (layers F.Cu B.Cu) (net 8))
 (segment (start 157.2 101.1) (end 154.7 101.1) (width 2) (layer F.Cu) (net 8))
 (segment (start 153.6 89.1) (end 153.6 97.1) (width 2) (layer F.Cu) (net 8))
 (segment (start 153.6 97.1) (end 157.2 97.1) (width 2) (layer F.Cu) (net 8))
 (segment (start 157.2 109.2) (end 157.2 97.1) (width 2) (layer F.Cu) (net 8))
 (segment (start 158.3 82.3) (end 158.3 82.3) (width 2) (layer F.Cu) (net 19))
 (via (at 158.3 82.3) (size 2) (drill 1) (layers F.Cu B.Cu) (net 19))
 (segment (start 160.8 82.3) (end 158.3 82.3) (width 2) (layer F.Cu) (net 19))
 (segment (start 160.8 86.3) (end 160.8 74.2) (width 2) (layer F.Cu) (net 19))
 (segment (start 157.2 94.3) (end 157.2 86.4) (width 2) (layer F.Cu) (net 19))
 (segment (start 157.3 86.3) (end 160.8 86.3) (width 2) (layer F.Cu) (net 19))
 (segment (start 157.2 86.4) (end 157.3 86.3) (width 2) (layer F.Cu) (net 19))
 (segment (start 161.9 101.1) (end 161.9 101.1) (width 2) (layer F.Cu) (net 7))
 (via (at 161.9 101.1) (size 2) (drill 1) (layers F.Cu B.Cu) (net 7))
 (segment (start 164.4 101.1) (end 161.9 101.1) (width 2) (layer F.Cu) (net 7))
 (segment (start 160.8 89.1) (end 160.8 97.1) (width 2) (layer F.Cu) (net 7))
 (segment (start 160.8 97.1) (end 164.4 97.1) (width 2) (layer F.Cu) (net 7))
 (segment (start 164.4 109.2) (end 164.4 97.1) (width 2) (layer F.Cu) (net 7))
 (segment (start 165.5 82.3) (end 165.5 82.3) (width 2) (layer F.Cu) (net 18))
 (via (at 165.5 82.3) (size 2) (drill 1) (layers F.Cu B.Cu) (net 18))
 (segment (start 168 82.3) (end 165.5 82.3) (width 2) (layer F.Cu) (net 18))
 (segment (start 168 74.2) (end 168 86.3) (width 2) (layer F.Cu) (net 18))
 (segment (start 164.4 94.3) (end 164.4 86.3) (width 2) (layer F.Cu) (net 18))
 (segment (start 164.4 86.3) (end 168 86.3) (width 2) (layer F.Cu) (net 18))
 (segment (start 169.1 101.1) (end 169.1 101.1) (width 2) (layer F.Cu) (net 6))
 (via (at 169.1 101.1) (size 2) (drill 1) (layers F.Cu B.Cu) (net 6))
 (segment (start 171.6 101.1) (end 169.1 101.1) (width 2) (layer F.Cu) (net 6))
 (segment (start 168 89.1) (end 168 97.1) (width 2) (layer F.Cu) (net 6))
 (segment (start 168 97.1) (end 171.6 97.1) (width 2) (layer F.Cu) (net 6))
 (segment (start 171.6 97.1) (end 171.6 109.2) (width 2) (layer F.Cu) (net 6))
 (segment (start 172.7 82.3) (end 172.7 82.3) (width 2) (layer F.Cu) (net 28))
 (via (at 172.7 82.3) (size 2) (drill 1) (layers F.Cu B.Cu) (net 28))
 (segment (start 175.2 82.3) (end 172.7 82.3) (width 2) (layer F.Cu) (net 28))
 (segment (start 175.2 86.3) (end 175.2 74.2) (width 2) (layer F.Cu) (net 28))
 (segment (start 171.6 94.3) (end 171.6 86.3) (width 2) (layer F.Cu) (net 28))
 (segment (start 171.6 86.3) (end 175.2 86.3) (width 2) (layer F.Cu) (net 28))
 (segment (start 176.3 101.1) (end 176.3 101.1) (width 2) (layer F.Cu) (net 5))
 (via (at 176.3 101.1) (size 2) (drill 1) (layers F.Cu B.Cu) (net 5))
 (segment (start 178.8 101.1) (end 176.3 101.1) (width 2) (layer F.Cu) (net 5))
 (segment (start 175.2 89.1) (end 175.2 97.1) (width 2) (layer F.Cu) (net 5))
 (segment (start 175.2 97.1) (end 178.8 97.1) (width 2) (layer F.Cu) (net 5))
 (segment (start 178.8 97.1) (end 178.8 109.2) (width 2) (layer F.Cu) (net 5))
 (segment (start 179.9 82.3) (end 179.9 82.3) (width 2) (layer F.Cu) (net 17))
 (via (at 179.9 82.3) (size 2) (drill 1) (layers F.Cu B.Cu) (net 17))
 (segment (start 182.4 82.3) (end 179.9 82.3) (width 2) (layer F.Cu) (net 17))
 (segment (start 178.8 94.3) (end 178.8 86.3) (width 2) (layer F.Cu) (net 17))
 (segment (start 178.8 86.3) (end 182.4 86.3) (width 2) (layer F.Cu) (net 17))
 (segment (start 182.4 86.3) (end 182.4 74.2) (width 2) (layer F.Cu) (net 17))
 (segment (start 183.5 101.1) (end 183.5 101.1) (width 2) (layer F.Cu) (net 4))
 (via (at 183.5 101.1) (size 2) (drill 1) (layers F.Cu B.Cu) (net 4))
 (segment (start 186 101.1) (end 183.5 101.1) (width 2) (layer F.Cu) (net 4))
 (segment (start 182.4 89.1) (end 182.4 97.1) (width 2) (layer F.Cu) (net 4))
 (segment (start 182.4 97.1) (end 186 97.1) (width 2) (layer F.Cu) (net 4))
 (segment (start 186 97.1) (end 186 109.2) (width 2) (layer F.Cu) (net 4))
 (segment (start 187.1 82.3) (end 187.1 82.3) (width 2) (layer F.Cu) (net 16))
 (via (at 187.1 82.3) (size 2) (drill 1) (layers F.Cu B.Cu) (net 16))
 (segment (start 189.6 82.3) (end 187.1 82.3) (width 2) (layer F.Cu) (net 16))
 (segment (start 186 94.3) (end 186 86.3) (width 2) (layer F.Cu) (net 16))
 (segment (start 186 86.3) (end 189.6 86.3) (width 2) (layer F.Cu) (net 16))
 (segment (start 189.6 86.3) (end 189.6 74.2) (width 2) (layer F.Cu) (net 16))
 (segment (start 190.7 101.1) (end 190.7 101.1) (width 2) (layer F.Cu) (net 3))
 (via (at 190.7 101.1) (size 2) (drill 1) (layers F.Cu B.Cu) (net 3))
 (segment (start 193.2 101.1) (end 190.7 101.1) (width 2) (layer F.Cu) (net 3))
 (segment (start 189.6 89.1) (end 189.6 97.1) (width 2) (layer F.Cu) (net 3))
 (segment (start 189.6 97.1) (end 193.2 97.1) (width 2) (layer F.Cu) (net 3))
 (segment (start 193.2 97.1) (end 193.2 109.1) (width 2) (layer F.Cu) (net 3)))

